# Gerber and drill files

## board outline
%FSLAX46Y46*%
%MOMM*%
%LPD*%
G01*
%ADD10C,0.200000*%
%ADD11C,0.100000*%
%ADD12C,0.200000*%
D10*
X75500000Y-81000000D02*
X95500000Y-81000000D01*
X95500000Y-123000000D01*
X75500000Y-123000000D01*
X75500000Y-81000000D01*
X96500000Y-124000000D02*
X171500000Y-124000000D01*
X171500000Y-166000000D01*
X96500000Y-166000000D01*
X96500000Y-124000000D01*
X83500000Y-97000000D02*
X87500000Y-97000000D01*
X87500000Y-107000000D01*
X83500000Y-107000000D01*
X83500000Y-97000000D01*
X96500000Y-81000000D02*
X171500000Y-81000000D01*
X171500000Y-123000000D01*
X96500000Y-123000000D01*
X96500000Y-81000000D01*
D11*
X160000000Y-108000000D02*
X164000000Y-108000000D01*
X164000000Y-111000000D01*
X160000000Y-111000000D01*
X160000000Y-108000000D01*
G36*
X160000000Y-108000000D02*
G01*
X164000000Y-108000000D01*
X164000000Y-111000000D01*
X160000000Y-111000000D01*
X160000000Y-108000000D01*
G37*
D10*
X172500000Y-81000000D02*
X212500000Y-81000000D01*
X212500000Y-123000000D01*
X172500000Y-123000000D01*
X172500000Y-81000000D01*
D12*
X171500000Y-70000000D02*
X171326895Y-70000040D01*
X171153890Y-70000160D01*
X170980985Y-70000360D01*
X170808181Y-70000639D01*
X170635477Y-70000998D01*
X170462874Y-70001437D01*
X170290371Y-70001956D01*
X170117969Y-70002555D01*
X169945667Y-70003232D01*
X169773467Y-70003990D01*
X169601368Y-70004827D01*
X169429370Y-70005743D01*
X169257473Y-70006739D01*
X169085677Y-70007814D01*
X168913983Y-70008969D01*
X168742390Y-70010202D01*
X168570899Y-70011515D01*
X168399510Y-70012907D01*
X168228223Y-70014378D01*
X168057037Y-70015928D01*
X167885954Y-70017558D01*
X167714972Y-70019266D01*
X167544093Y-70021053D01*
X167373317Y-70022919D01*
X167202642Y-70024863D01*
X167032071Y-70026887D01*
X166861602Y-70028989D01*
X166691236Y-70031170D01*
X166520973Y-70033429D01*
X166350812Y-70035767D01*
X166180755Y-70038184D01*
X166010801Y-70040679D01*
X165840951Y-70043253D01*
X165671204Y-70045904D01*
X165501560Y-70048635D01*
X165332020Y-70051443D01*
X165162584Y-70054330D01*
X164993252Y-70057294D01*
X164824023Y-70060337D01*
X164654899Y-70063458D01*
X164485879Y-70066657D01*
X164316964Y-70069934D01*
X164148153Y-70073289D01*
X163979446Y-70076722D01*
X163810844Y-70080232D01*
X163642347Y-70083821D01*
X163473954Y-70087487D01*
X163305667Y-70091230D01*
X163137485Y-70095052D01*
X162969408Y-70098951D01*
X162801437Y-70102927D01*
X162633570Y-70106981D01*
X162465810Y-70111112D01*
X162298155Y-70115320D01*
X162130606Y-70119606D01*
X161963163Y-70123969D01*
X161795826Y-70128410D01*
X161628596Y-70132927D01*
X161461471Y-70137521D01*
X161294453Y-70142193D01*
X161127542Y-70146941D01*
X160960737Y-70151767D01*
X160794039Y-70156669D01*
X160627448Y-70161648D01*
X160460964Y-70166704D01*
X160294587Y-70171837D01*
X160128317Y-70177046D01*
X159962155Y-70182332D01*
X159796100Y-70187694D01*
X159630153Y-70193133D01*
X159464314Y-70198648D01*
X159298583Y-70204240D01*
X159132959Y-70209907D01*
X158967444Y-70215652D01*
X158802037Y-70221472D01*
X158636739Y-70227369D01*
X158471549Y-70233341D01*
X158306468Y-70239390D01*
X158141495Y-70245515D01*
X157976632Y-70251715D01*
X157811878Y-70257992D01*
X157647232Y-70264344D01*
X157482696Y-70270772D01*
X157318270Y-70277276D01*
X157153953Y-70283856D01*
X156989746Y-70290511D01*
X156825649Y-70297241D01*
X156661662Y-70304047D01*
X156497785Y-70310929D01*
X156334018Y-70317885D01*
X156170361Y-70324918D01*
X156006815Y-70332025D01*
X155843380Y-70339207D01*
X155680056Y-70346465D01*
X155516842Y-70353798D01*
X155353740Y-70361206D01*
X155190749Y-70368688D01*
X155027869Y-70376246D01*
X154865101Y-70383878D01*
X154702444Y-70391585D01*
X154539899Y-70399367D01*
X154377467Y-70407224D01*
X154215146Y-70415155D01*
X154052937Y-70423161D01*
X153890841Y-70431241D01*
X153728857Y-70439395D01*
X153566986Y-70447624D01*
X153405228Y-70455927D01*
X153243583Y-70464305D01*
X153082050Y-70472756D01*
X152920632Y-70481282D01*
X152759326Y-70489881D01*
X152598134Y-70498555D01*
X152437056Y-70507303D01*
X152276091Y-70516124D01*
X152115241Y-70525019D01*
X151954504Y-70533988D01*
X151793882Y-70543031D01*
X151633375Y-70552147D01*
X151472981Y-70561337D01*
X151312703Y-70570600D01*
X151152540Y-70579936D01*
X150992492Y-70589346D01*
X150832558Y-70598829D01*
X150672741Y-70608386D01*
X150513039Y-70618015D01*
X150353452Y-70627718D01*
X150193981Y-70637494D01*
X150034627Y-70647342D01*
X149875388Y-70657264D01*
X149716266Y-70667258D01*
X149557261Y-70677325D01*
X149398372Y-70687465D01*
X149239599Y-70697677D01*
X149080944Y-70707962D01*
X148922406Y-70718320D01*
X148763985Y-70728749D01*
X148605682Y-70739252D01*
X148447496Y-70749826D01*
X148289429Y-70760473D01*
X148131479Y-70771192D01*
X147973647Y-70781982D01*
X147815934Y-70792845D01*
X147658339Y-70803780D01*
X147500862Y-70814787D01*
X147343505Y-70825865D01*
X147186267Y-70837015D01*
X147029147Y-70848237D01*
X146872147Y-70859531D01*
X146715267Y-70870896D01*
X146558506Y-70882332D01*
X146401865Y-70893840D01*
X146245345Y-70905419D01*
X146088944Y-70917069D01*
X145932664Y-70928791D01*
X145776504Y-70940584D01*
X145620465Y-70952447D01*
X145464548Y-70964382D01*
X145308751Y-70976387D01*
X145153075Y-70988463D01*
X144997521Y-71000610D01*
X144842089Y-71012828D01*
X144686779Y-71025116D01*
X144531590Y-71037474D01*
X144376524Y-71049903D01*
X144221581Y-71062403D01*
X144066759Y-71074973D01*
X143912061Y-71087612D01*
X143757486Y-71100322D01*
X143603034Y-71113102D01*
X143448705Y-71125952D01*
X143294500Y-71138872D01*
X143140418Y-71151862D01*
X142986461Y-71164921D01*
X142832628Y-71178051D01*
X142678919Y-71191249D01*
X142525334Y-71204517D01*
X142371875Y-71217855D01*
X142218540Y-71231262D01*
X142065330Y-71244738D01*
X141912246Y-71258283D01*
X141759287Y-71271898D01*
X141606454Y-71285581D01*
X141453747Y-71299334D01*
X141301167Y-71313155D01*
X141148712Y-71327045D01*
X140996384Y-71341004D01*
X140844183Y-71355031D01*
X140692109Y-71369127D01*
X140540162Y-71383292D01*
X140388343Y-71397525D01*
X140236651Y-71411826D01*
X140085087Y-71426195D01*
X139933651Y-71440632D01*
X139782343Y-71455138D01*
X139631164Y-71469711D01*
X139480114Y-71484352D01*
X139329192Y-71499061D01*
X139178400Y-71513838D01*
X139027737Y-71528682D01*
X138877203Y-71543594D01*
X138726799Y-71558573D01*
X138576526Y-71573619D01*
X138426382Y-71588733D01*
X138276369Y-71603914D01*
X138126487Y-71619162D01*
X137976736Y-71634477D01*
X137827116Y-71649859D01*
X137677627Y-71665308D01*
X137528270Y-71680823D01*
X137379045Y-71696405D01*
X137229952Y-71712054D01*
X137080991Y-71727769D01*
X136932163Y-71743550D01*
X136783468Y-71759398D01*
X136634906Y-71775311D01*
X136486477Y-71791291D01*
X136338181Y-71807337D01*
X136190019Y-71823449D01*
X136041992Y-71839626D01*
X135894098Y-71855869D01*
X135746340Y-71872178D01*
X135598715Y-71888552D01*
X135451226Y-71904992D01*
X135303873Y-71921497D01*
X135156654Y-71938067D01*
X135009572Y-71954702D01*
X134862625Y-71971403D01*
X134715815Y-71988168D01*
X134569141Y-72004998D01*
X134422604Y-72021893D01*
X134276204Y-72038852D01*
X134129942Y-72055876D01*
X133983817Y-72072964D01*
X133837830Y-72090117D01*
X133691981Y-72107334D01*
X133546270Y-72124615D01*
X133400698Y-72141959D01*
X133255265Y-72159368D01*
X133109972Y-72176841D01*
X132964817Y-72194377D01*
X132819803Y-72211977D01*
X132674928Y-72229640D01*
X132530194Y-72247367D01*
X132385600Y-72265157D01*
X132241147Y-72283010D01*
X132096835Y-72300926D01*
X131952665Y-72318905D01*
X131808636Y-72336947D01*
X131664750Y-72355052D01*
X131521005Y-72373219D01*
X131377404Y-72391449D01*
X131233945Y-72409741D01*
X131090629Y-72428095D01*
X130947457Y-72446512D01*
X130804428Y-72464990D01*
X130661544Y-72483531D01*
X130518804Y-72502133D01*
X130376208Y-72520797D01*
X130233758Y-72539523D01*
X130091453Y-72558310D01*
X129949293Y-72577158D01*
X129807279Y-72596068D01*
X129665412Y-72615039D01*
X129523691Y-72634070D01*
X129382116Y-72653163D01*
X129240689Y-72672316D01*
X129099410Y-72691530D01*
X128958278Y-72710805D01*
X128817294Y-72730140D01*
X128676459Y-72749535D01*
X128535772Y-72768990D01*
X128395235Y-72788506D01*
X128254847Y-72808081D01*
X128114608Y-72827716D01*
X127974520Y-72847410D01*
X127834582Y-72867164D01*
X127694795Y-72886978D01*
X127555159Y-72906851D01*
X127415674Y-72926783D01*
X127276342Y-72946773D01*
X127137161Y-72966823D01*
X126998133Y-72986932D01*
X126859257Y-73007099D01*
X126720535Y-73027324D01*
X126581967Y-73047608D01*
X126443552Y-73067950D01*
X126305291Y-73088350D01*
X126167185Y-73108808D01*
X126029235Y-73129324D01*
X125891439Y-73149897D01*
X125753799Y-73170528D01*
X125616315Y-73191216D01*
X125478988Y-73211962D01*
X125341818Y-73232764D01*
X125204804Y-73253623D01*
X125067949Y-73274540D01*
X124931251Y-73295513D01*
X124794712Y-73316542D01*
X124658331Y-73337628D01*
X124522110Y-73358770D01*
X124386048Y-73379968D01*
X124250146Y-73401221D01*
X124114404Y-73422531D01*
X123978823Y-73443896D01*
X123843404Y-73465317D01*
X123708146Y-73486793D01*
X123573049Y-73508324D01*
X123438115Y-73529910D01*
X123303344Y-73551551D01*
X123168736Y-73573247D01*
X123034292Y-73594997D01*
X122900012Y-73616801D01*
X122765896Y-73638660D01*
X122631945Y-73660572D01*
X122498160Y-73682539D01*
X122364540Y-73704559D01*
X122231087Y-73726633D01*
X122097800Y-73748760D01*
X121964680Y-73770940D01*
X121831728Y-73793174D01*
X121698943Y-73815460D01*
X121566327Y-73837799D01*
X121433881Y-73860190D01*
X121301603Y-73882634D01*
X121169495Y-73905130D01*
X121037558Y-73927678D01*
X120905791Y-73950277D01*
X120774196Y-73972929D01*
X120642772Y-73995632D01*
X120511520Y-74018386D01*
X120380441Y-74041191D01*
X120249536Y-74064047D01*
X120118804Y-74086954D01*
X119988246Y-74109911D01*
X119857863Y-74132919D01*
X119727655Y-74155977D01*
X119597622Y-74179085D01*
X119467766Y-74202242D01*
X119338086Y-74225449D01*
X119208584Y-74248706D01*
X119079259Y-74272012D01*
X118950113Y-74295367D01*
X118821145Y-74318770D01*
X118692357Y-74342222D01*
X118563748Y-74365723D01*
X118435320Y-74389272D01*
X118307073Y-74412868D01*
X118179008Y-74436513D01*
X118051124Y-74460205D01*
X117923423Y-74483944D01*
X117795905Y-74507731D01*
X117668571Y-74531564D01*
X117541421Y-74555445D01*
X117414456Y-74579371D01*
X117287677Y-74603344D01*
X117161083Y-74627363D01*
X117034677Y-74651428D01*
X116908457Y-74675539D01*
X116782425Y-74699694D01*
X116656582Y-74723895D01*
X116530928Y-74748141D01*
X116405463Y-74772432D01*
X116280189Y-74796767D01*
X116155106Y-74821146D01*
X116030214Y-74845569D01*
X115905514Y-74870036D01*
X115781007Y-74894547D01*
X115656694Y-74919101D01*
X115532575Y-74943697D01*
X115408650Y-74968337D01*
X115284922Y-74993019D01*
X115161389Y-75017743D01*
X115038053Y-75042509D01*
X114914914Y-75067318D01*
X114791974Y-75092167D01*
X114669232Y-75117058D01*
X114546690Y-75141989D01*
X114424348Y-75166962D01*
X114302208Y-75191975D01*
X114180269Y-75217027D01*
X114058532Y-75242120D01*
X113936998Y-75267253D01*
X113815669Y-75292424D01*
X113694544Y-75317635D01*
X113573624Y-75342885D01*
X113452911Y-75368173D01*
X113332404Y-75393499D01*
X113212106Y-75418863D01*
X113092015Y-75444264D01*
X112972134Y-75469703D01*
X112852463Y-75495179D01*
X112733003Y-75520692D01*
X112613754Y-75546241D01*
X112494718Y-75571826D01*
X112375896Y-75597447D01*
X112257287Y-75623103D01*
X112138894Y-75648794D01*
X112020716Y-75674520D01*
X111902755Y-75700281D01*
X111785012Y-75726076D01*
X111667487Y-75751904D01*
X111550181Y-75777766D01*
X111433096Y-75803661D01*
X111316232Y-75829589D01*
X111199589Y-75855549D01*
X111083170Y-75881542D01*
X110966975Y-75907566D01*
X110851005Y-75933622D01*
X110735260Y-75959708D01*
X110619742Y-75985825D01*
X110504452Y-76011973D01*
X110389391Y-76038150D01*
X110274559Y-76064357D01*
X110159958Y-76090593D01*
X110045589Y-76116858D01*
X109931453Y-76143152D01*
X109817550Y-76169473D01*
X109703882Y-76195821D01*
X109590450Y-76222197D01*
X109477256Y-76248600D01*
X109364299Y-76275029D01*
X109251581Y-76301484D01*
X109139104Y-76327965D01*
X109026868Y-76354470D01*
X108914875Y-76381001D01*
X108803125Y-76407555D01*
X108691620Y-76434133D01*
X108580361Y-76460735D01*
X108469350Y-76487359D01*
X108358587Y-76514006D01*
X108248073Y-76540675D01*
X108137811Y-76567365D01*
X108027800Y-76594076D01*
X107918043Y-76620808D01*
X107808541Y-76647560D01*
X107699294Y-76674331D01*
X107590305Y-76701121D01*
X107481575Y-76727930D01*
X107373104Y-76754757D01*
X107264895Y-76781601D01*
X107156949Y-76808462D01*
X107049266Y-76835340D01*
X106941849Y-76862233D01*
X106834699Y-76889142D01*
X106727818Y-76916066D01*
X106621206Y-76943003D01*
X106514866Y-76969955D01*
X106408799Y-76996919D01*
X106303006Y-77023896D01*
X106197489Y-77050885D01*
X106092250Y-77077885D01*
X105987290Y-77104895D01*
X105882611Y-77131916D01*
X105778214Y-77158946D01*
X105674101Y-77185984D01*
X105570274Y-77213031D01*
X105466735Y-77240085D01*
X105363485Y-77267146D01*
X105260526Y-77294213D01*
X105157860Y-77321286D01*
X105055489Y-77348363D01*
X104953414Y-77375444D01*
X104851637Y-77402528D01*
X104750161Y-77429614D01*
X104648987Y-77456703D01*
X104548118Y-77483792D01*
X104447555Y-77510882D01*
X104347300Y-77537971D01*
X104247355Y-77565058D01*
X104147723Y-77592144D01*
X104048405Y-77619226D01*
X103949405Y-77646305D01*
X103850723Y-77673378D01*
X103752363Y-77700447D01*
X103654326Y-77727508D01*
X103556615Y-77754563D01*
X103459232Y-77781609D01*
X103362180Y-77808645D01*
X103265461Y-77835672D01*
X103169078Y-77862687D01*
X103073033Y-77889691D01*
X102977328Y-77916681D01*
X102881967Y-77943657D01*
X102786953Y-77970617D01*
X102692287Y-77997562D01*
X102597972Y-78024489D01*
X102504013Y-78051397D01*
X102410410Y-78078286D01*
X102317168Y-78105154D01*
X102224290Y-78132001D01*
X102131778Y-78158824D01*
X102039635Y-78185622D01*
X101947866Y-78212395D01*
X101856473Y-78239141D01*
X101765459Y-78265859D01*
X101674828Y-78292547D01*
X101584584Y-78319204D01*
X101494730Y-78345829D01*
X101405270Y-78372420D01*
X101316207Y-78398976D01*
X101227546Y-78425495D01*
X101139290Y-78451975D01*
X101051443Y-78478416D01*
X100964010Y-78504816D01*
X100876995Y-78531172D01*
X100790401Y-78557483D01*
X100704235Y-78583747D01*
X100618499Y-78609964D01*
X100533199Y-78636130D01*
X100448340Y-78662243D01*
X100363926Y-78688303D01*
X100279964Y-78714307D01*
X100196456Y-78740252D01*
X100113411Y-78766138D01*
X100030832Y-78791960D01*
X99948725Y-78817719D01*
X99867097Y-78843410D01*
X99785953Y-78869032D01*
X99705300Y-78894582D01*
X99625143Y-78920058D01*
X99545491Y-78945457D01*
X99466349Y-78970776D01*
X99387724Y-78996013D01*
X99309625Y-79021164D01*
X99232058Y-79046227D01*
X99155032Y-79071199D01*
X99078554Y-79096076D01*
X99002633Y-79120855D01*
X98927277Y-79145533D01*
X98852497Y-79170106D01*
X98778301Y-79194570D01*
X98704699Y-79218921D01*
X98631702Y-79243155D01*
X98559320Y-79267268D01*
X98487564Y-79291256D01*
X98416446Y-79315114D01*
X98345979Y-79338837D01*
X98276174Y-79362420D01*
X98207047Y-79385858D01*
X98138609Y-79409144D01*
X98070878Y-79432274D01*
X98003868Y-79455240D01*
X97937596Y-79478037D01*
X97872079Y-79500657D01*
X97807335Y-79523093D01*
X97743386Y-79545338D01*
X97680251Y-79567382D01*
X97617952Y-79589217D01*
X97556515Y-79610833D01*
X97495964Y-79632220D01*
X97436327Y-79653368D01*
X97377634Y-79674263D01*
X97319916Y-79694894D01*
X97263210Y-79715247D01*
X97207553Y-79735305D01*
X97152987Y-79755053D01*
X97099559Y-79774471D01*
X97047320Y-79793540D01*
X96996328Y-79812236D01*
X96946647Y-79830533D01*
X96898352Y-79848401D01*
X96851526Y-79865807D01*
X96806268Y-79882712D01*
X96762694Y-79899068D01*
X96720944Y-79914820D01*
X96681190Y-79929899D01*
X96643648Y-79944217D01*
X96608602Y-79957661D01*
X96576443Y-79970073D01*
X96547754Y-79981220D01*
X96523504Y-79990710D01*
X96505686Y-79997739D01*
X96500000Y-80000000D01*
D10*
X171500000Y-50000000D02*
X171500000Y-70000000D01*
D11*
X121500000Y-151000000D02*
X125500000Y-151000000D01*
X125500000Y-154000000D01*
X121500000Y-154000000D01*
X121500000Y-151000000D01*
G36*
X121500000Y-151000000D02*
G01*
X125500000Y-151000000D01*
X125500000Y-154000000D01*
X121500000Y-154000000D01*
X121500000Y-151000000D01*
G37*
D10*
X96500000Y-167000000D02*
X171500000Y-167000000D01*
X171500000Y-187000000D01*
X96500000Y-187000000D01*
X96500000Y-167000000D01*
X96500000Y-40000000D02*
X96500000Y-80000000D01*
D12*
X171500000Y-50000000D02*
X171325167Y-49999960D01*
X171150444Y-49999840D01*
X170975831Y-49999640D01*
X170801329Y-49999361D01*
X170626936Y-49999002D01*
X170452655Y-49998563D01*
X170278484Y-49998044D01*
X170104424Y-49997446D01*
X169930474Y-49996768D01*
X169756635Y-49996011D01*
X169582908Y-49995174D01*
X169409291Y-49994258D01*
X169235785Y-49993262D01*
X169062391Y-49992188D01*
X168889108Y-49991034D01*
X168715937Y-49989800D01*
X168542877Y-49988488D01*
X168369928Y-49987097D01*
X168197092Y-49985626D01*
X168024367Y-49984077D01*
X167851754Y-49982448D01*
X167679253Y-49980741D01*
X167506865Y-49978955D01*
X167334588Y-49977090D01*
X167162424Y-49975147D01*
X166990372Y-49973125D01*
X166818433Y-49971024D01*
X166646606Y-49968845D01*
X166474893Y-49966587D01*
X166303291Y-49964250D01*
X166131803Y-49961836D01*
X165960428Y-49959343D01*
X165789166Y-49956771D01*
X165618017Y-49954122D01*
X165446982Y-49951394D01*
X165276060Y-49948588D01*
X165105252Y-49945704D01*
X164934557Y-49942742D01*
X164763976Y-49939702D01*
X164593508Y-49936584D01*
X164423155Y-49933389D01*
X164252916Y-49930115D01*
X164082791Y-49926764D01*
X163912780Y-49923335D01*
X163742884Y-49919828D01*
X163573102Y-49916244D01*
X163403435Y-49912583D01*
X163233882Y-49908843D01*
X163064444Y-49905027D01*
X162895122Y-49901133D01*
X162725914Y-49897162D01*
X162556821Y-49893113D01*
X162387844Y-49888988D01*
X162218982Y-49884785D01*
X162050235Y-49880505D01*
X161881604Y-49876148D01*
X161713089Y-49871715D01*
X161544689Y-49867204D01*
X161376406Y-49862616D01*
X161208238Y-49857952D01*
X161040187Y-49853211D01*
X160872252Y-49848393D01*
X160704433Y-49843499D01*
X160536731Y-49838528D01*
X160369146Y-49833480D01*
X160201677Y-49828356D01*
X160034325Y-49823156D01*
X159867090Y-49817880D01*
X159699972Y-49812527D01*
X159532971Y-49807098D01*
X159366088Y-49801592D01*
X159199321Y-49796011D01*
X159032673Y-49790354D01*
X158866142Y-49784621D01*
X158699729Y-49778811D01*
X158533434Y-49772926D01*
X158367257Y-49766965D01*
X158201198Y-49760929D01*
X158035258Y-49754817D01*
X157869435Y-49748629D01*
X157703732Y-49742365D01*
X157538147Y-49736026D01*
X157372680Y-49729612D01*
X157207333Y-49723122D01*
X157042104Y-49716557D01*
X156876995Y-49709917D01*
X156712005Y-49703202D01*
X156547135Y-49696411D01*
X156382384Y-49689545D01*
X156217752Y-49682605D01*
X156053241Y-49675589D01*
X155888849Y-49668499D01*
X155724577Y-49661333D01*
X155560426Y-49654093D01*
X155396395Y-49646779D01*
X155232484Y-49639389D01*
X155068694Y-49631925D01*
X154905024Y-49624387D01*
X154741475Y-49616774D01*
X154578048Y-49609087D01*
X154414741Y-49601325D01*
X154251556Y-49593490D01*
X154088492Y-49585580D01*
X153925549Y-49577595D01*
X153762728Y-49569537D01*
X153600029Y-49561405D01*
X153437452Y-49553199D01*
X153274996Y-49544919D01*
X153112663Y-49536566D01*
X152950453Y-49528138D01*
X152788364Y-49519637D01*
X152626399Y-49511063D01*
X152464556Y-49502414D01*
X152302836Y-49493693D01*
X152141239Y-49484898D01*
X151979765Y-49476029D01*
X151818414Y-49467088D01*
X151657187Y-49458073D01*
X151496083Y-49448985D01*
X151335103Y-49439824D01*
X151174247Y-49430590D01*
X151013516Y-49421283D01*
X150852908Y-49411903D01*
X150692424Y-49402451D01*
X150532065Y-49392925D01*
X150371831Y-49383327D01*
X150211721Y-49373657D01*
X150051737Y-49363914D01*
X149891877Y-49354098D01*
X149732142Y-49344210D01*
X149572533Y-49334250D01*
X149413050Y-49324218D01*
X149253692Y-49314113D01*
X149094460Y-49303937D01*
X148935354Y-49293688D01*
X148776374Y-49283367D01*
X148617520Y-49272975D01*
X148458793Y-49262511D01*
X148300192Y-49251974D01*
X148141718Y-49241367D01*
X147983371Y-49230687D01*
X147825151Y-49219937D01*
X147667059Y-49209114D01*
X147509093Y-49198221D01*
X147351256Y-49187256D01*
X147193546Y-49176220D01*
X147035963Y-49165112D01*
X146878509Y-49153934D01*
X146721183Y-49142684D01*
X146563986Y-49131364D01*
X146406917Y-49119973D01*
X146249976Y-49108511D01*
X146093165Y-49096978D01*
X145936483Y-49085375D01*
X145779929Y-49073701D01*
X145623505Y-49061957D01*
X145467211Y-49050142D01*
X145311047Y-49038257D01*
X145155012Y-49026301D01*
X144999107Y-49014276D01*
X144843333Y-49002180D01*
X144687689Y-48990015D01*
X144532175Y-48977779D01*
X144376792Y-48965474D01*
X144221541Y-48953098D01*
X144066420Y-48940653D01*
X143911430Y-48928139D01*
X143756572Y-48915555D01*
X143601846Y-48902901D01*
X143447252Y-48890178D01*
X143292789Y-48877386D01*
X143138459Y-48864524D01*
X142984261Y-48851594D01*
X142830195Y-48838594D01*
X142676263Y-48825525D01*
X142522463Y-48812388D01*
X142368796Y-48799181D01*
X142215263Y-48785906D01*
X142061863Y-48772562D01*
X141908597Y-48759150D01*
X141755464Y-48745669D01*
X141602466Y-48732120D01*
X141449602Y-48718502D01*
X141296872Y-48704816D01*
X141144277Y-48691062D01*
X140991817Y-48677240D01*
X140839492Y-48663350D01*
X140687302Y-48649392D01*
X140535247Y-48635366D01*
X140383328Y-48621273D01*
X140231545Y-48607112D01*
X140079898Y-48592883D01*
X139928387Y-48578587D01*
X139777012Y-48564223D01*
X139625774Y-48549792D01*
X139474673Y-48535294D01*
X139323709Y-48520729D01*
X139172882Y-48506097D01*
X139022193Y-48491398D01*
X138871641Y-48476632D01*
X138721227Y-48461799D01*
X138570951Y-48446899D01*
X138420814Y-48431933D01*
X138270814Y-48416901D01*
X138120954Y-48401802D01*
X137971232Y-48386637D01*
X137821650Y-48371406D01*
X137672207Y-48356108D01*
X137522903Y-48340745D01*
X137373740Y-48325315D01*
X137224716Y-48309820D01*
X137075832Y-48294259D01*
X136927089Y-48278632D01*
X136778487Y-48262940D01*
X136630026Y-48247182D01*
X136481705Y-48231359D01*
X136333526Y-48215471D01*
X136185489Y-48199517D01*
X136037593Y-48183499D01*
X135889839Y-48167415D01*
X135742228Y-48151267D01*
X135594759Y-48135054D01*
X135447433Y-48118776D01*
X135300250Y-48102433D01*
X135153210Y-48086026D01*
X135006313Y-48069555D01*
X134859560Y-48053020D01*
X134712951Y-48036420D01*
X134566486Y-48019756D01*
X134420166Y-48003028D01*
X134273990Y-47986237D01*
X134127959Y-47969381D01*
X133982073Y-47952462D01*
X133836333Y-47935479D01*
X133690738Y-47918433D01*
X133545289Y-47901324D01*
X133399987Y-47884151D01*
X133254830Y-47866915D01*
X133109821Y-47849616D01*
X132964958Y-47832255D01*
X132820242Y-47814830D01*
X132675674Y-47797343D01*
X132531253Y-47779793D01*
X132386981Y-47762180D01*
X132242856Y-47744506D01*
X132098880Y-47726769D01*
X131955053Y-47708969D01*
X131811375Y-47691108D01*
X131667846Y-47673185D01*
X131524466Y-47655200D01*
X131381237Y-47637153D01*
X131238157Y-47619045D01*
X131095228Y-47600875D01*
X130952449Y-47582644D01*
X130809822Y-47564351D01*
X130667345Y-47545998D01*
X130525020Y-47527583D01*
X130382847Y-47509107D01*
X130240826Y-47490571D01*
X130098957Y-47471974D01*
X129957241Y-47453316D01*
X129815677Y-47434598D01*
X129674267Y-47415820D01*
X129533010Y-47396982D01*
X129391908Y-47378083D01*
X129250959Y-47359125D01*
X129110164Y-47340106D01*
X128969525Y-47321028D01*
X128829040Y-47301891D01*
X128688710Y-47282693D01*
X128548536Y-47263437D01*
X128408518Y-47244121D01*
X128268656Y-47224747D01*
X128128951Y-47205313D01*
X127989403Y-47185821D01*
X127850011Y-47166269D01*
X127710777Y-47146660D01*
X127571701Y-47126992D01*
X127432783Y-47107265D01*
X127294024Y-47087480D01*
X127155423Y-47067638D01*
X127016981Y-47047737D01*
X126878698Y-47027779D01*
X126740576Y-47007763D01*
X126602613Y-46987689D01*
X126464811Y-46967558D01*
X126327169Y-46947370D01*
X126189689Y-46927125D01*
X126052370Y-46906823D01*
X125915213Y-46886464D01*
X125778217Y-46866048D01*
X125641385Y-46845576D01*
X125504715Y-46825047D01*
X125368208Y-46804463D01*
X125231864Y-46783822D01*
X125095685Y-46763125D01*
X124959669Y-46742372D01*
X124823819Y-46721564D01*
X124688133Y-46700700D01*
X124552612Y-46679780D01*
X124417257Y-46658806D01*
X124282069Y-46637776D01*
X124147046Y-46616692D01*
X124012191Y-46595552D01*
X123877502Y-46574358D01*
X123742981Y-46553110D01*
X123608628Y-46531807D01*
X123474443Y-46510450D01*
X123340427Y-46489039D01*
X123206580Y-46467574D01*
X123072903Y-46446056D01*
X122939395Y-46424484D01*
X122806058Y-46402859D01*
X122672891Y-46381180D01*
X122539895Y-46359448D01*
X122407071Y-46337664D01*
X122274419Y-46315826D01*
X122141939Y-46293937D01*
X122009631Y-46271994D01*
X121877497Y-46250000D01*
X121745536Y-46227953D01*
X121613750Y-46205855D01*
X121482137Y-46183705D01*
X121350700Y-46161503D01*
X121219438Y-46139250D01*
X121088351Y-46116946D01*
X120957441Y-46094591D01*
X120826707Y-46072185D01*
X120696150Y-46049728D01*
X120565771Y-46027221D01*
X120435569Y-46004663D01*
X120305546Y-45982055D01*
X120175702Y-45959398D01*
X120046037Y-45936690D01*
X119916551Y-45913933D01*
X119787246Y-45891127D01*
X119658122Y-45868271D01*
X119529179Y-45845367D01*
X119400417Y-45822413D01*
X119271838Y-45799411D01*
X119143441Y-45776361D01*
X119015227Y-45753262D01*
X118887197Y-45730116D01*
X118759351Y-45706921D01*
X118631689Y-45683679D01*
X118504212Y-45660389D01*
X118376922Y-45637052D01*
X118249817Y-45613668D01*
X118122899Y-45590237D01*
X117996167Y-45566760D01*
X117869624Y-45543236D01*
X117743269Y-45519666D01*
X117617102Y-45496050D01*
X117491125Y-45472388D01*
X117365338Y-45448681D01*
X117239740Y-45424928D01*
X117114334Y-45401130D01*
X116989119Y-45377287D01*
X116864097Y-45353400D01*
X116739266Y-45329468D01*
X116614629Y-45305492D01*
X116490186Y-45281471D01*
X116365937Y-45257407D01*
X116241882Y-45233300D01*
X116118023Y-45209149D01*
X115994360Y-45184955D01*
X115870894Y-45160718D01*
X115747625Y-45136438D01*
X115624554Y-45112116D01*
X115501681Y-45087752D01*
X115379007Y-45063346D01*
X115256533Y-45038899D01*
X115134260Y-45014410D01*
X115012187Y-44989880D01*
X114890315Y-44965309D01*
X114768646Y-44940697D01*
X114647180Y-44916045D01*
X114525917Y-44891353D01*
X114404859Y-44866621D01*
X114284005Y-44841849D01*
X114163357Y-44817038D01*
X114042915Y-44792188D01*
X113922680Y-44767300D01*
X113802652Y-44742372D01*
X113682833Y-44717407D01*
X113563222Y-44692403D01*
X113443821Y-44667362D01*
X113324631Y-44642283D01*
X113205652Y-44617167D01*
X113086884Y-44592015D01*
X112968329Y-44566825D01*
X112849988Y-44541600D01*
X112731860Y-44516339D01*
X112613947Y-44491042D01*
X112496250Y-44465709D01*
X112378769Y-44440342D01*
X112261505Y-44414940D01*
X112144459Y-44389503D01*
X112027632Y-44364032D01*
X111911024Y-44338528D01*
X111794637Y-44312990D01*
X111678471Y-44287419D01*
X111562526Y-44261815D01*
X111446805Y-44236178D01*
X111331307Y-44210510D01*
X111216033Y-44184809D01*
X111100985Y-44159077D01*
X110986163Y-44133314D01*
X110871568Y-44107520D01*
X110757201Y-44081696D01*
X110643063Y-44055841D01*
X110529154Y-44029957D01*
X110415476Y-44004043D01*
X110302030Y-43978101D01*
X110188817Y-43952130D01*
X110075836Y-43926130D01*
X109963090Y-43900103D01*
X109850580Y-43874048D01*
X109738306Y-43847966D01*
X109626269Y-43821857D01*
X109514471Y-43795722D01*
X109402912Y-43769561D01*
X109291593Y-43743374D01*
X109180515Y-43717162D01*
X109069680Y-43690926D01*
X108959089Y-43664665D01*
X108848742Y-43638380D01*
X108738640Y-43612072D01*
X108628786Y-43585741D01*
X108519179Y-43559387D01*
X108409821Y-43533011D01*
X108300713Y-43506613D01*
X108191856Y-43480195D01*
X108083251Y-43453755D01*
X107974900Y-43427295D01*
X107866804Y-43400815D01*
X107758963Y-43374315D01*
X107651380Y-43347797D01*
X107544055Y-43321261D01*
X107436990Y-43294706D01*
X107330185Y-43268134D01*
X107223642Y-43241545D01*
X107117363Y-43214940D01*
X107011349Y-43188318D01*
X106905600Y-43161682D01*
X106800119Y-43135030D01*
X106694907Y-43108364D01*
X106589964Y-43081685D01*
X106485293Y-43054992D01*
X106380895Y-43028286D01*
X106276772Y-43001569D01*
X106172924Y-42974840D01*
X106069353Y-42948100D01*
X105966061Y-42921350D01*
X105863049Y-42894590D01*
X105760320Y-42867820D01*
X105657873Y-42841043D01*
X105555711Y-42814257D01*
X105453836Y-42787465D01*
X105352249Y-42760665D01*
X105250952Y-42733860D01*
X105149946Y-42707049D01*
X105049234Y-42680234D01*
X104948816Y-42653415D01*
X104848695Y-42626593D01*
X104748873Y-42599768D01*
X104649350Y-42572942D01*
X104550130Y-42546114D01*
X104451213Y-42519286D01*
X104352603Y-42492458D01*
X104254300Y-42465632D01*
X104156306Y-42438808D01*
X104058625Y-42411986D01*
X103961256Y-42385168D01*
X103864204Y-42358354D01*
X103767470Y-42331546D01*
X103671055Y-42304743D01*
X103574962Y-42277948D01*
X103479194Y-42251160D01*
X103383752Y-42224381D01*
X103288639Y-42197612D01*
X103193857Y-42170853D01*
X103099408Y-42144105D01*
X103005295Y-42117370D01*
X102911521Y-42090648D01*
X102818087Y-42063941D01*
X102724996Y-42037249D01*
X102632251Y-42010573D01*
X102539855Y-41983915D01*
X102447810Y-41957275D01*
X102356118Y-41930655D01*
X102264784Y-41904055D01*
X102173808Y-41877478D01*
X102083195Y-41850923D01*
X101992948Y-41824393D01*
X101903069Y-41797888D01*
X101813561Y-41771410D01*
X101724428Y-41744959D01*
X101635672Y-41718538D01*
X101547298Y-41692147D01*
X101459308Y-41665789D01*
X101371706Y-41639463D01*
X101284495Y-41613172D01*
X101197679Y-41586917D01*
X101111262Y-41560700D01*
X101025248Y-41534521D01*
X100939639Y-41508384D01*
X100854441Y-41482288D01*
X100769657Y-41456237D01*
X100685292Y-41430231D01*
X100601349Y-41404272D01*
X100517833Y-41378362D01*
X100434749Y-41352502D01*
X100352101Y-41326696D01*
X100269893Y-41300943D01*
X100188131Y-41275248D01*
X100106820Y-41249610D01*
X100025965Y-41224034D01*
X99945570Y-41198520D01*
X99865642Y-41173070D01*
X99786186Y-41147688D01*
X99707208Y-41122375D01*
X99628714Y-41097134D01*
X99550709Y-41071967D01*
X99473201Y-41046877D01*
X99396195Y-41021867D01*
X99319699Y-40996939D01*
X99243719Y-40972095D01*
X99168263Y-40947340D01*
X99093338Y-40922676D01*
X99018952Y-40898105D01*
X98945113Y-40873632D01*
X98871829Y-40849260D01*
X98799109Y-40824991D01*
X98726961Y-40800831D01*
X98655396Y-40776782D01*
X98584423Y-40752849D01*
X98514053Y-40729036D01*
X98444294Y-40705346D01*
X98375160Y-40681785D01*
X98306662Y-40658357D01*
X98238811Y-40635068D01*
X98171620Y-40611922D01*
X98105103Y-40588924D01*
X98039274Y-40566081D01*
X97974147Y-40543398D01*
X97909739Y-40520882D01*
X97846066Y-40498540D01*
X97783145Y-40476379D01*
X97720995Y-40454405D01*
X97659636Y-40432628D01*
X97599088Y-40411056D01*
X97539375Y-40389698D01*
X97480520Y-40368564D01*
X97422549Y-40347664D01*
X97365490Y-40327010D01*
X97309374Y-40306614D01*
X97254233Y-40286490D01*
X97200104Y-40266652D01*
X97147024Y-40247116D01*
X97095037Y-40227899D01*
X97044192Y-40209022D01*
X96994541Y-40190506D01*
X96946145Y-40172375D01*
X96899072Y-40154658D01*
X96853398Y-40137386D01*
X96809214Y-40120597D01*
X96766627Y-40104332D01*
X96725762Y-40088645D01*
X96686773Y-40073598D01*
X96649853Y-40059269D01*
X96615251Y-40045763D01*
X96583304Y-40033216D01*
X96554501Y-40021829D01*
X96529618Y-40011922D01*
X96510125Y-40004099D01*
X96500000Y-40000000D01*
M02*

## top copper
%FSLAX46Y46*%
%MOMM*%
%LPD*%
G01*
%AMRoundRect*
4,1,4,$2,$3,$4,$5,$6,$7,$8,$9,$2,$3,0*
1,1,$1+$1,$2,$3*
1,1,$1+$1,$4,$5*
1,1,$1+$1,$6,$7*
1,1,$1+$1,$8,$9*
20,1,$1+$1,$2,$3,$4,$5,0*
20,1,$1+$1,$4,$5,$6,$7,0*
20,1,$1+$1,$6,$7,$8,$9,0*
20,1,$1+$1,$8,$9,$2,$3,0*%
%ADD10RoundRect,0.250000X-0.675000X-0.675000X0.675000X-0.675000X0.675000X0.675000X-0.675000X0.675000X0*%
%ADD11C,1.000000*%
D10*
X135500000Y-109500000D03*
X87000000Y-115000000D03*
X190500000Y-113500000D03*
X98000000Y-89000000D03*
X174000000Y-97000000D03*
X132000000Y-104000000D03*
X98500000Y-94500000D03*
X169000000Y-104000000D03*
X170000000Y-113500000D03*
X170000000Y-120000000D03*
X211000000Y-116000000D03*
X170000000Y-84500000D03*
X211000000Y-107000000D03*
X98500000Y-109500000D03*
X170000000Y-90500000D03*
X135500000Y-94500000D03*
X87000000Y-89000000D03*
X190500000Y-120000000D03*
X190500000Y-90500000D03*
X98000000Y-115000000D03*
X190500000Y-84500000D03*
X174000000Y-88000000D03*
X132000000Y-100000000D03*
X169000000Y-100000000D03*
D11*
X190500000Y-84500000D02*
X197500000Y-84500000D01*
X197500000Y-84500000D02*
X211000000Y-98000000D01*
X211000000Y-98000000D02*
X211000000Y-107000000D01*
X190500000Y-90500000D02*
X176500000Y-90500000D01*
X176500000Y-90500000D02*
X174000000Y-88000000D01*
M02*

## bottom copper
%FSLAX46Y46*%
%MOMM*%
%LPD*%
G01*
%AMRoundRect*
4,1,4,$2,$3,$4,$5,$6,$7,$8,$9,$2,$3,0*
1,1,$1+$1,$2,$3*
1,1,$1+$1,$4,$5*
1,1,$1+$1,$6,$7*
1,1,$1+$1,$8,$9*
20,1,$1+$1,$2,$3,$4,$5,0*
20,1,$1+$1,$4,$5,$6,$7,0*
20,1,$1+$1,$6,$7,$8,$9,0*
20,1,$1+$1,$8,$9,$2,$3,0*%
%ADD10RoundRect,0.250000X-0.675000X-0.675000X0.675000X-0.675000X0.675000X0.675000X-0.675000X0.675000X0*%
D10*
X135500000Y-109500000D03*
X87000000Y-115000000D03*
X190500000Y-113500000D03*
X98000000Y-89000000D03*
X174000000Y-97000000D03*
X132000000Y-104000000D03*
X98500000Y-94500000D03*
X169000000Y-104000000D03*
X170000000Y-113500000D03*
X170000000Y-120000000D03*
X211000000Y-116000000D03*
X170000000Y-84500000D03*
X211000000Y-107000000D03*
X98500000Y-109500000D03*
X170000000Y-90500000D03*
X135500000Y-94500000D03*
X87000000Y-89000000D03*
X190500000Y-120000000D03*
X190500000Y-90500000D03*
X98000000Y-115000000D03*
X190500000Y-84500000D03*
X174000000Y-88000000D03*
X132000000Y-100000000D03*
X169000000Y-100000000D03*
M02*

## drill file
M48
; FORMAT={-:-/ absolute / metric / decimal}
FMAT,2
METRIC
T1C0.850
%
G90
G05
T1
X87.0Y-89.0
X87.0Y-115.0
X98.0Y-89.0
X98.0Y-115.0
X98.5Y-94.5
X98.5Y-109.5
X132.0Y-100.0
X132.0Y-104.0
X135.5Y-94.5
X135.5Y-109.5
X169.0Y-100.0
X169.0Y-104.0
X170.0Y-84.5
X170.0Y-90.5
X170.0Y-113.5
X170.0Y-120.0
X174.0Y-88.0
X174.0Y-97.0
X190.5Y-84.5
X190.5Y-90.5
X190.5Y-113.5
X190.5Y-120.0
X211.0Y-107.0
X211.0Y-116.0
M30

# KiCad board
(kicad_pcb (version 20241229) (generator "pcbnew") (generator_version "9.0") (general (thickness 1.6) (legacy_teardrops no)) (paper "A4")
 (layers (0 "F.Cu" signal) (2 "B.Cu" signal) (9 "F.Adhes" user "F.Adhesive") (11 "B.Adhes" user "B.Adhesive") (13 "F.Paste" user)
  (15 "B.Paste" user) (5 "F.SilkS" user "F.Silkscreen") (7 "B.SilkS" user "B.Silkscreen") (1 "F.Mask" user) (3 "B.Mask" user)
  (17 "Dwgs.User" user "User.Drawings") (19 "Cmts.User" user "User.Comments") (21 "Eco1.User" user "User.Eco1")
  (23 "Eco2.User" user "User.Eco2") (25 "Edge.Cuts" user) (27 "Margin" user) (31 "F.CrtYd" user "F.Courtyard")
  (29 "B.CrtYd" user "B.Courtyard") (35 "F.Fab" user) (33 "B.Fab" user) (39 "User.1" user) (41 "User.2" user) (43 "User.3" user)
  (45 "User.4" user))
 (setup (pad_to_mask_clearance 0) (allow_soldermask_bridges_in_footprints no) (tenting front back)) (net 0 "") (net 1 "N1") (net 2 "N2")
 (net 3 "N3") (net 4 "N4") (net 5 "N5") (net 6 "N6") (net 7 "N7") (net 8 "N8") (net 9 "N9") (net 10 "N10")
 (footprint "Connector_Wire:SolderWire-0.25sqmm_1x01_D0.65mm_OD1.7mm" (layer "F.Cu") (at 135.5 109.5)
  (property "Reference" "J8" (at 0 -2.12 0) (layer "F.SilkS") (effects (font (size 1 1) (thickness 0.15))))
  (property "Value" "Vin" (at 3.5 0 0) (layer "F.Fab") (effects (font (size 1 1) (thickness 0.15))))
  (pad "1" thru_hole roundrect (at 0 0) (size 1.85 1.85) (drill 0.85) (layers "*.Cu" "*.Mask") (remove_unused_layers no)
   (roundrect_rratio 0.135135) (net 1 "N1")))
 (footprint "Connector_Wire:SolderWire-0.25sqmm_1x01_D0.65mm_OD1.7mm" (layer "F.Cu") (at 87 115)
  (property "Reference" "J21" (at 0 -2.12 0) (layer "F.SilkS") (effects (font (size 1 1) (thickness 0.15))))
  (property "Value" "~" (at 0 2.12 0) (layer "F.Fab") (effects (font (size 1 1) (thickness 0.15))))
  (pad "1" thru_hole roundrect (at 0 0) (size 1.85 1.85) (drill 0.85) (layers "*.Cu" "*.Mask") (remove_unused_layers no)
   (roundrect_rratio 0.135135) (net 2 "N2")))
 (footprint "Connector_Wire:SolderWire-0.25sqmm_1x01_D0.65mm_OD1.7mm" (layer "F.Cu") (at 190.5 113.5)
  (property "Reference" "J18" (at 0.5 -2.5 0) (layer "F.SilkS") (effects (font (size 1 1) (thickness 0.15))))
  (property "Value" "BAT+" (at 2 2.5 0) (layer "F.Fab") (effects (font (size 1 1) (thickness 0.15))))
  (pad "1" thru_hole roundrect (at 0 0) (size 1.85 1.85) (drill 0.85) (layers "*.Cu" "*.Mask") (remove_unused_layers no)
   (roundrect_rratio 0.135135) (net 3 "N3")))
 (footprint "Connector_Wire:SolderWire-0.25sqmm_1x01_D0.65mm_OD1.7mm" (layer "F.Cu") (at 98 89)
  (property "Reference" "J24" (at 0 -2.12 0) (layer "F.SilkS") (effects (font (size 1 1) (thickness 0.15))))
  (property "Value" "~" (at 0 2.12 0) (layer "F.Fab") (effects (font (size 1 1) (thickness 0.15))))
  (pad "1" thru_hole roundrect (at 0 0) (size 1.85 1.85) (drill 0.85) (layers "*.Cu" "*.Mask") (remove_unused_layers no)
   (roundrect_rratio 0.135135) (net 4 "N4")))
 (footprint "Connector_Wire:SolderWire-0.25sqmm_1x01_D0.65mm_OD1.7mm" (layer "F.Cu") (at 174 97)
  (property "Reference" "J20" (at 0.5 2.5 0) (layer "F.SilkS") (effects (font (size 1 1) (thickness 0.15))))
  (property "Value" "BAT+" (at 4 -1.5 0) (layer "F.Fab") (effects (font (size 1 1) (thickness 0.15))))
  (pad "1" thru_hole roundrect (at 0 0) (size 1.85 1.85) (drill 0.85) (layers "*.Cu" "*.Mask") (remove_unused_layers no)
   (roundrect_rratio 0.135135) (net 3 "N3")))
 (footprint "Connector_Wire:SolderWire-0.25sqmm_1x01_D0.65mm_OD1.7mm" (layer "F.Cu") (at 132 104)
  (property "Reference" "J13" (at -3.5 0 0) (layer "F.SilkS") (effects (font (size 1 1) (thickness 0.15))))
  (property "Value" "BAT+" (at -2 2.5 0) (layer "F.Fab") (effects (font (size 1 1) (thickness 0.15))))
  (pad "1" thru_hole roundrect (at 0 0) (size 1.85 1.85) (drill 0.85) (layers "*.Cu" "*.Mask") (remove_unused_layers no)
   (roundrect_rratio 0.135135) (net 3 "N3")))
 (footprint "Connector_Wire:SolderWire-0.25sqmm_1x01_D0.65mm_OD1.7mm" (layer "F.Cu") (at 98.5 94.5)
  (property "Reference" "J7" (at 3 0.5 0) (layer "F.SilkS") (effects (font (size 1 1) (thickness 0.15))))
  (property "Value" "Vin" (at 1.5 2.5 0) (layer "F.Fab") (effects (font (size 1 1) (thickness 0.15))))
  (pad "1" thru_hole roundrect (at 0 0) (size 1.85 1.85) (drill 0.85) (layers "*.Cu" "*.Mask") (remove_unused_layers no)
   (roundrect_rratio 0.135135) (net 1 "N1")))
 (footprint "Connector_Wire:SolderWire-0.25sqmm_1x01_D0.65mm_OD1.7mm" (layer "F.Cu") (at 169 104)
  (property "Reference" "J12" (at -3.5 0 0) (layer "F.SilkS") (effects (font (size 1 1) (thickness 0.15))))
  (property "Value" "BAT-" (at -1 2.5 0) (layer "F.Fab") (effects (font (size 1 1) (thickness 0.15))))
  (pad "1" thru_hole roundrect (at 0 0) (size 1.85 1.85) (drill 0.85) (layers "*.Cu" "*.Mask") (remove_unused_layers no)
   (roundrect_rratio 0.135135) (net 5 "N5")))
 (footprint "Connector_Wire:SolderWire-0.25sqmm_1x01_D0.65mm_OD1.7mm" (layer "F.Cu") (at 170 113.5)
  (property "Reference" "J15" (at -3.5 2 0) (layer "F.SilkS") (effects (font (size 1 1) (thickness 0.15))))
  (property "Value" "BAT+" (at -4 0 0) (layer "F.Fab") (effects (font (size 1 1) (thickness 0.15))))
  (pad "1" thru_hole roundrect (at 0 0) (size 1.85 1.85) (drill 0.85) (layers "*.Cu" "*.Mask") (remove_unused_layers no)
   (roundrect_rratio 0.135135) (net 3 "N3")))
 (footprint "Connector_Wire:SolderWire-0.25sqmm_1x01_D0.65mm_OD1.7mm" (layer "F.Cu") (at 170 120)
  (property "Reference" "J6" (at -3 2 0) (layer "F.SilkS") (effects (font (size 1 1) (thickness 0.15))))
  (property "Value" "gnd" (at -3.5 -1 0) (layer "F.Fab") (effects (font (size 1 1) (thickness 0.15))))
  (pad "1" thru_hole roundrect (at 0 0) (size 1.85 1.85) (drill 0.85) (layers "*.Cu" "*.Mask") (remove_unused_layers no)
   (roundrect_rratio 0.135135) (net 5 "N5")))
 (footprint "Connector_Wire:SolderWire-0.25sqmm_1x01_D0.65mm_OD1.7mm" (layer "F.Cu") (at 211 116)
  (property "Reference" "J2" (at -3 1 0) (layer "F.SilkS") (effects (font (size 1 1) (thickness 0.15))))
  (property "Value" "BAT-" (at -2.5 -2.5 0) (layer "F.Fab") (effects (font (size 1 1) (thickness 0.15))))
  (pad "1" thru_hole roundrect (at 0 0) (size 1.85 1.85) (drill 0.85) (layers "*.Cu" "*.Mask") (remove_unused_layers no)
   (roundrect_rratio 0.135135) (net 5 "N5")))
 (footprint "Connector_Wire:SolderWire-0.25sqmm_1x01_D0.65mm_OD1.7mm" (layer "F.Cu") (at 170 84.5)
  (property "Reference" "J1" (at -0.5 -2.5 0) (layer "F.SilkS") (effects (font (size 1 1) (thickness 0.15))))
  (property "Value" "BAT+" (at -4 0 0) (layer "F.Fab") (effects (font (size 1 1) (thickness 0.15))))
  (pad "1" thru_hole roundrect (at 0 0) (size 1.85 1.85) (drill 0.85) (layers "*.Cu" "*.Mask") (remove_unused_layers no)
   (roundrect_rratio 0.135135) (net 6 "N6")))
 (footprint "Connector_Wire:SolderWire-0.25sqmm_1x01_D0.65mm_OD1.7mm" (layer "F.Cu") (at 211 107)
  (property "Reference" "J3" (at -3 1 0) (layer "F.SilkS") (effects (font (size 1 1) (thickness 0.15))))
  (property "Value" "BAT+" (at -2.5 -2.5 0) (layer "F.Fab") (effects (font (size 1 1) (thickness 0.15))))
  (pad "1" thru_hole roundrect (at 0 0) (size 1.85 1.85) (drill 0.85) (layers "*.Cu" "*.Mask") (remove_unused_layers no)
   (roundrect_rratio 0.135135) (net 6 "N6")))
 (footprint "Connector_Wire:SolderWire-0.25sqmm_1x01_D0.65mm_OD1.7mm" (layer "F.Cu") (at 98.5 109.5)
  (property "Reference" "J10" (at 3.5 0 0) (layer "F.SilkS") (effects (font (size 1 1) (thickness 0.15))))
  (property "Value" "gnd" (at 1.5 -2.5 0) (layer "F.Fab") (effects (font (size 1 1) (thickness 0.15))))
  (pad "1" thru_hole roundrect (at 0 0) (size 1.85 1.85) (drill 0.85) (layers "*.Cu" "*.Mask") (remove_unused_layers no)
   (roundrect_rratio 0.135135) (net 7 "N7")))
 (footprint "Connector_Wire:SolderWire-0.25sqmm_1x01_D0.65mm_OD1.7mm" (layer "F.Cu") (at 170 90.5)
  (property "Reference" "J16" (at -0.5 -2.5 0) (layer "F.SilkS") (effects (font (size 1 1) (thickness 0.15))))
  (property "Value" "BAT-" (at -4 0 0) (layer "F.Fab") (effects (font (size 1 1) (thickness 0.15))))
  (pad "1" thru_hole roundrect (at 0 0) (size 1.85 1.85) (drill 0.85) (layers "*.Cu" "*.Mask") (remove_unused_layers no)
   (roundrect_rratio 0.135135) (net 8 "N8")))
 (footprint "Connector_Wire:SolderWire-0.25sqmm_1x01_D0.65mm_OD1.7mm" (layer "F.Cu") (at 135.5 94.5)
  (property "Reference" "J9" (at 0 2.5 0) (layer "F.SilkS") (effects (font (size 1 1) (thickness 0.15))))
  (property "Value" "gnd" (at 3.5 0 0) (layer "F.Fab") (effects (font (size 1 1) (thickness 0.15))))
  (pad "1" thru_hole roundrect (at 0 0) (size 1.85 1.85) (drill 0.85) (layers "*.Cu" "*.Mask") (remove_unused_layers no)
   (roundrect_rratio 0.135135) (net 7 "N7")))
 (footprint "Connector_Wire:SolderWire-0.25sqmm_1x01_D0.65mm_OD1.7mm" (layer "F.Cu") (at 87 89)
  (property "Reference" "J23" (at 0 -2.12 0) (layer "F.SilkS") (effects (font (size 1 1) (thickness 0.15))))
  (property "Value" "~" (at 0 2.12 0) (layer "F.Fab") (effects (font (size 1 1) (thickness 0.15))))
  (pad "1" thru_hole roundrect (at 0 0) (size 1.85 1.85) (drill 0.85) (layers "*.Cu" "*.Mask") (remove_unused_layers no)
   (roundrect_rratio 0.135135) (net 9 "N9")))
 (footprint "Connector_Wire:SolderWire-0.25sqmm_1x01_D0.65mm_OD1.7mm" (layer "F.Cu") (at 190.5 120)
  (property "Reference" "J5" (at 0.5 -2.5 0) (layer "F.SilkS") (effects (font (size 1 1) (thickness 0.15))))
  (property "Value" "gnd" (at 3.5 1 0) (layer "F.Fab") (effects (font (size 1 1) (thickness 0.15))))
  (pad "1" thru_hole roundrect (at 0 0) (size 1.85 1.85) (drill 0.85) (layers "*.Cu" "*.Mask") (remove_unused_layers no)
   (roundrect_rratio 0.135135) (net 5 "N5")))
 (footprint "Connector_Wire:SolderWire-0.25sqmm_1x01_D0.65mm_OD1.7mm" (layer "F.Cu") (at 190.5 90.5)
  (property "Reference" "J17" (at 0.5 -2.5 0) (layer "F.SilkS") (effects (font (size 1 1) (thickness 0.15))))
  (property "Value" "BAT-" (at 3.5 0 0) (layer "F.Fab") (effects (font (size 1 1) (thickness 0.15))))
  (pad "1" thru_hole roundrect (at 0 0) (size 1.85 1.85) (drill 0.85) (layers "*.Cu" "*.Mask") (remove_unused_layers no)
   (roundrect_rratio 0.135135) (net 8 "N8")))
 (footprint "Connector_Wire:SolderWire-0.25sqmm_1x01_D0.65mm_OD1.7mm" (layer "F.Cu") (at 98 115)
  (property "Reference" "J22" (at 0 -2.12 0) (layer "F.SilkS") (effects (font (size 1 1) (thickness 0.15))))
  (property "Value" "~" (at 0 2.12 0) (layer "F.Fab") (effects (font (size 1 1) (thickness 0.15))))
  (pad "1" thru_hole roundrect (at 0 0) (size 1.85 1.85) (drill 0.85) (layers "*.Cu" "*.Mask") (remove_unused_layers no)
   (roundrect_rratio 0.135135) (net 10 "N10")))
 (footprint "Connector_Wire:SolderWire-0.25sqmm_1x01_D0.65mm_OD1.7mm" (layer "F.Cu") (at 190.5 84.5)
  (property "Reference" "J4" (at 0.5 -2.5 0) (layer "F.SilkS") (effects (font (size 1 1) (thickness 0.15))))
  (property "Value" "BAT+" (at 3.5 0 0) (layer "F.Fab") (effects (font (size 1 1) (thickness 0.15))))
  (pad "1" thru_hole roundrect (at 0 0) (size 1.85 1.85) (drill 0.85) (layers "*.Cu" "*.Mask") (remove_unused_layers no)
   (roundrect_rratio 0.135135) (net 6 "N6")))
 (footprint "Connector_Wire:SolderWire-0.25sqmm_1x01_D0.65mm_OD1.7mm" (layer "F.Cu") (at 174 88)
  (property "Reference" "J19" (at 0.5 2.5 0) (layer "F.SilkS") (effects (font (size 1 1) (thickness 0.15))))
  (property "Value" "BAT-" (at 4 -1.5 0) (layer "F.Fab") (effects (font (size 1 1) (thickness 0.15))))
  (pad "1" thru_hole roundrect (at 0 0) (size 1.85 1.85) (drill 0.85) (layers "*.Cu" "*.Mask") (remove_unused_layers no)
   (roundrect_rratio 0.135135) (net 8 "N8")))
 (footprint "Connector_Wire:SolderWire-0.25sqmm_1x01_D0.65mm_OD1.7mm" (layer "F.Cu") (at 132 100)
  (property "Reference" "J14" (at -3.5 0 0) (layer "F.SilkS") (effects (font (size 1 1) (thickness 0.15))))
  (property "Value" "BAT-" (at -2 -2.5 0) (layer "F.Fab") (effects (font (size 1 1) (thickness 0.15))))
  (pad "1" thru_hole roundrect (at 0 0) (size 1.85 1.85) (drill 0.85) (layers "*.Cu" "*.Mask") (remove_unused_layers no)
   (roundrect_rratio 0.135135) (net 8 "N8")))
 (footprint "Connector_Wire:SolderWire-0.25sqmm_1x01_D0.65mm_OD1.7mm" (layer "F.Cu") (at 169 100)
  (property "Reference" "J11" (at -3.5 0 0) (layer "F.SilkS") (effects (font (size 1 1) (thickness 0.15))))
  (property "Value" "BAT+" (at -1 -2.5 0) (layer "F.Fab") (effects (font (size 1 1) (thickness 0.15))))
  (pad "1" thru_hole roundrect (at 0 0) (size 1.85 1.85) (drill 0.85) (layers "*.Cu" "*.Mask") (remove_unused_layers no)
   (roundrect_rratio 0.135135) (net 6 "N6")))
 (gr_rect (start 75.5 81) (end 95.5 123) (stroke (width 0.2) (type solid)) (fill no) (layer "Edge.Cuts"))
 (gr_rect (start 96.5 124) (end 171.5 166) (stroke (width 0.2) (type solid)) (fill no) (layer "Edge.Cuts"))
 (gr_rect (start 83.5 97) (end 87.5 107) (stroke (width 0.2) (type solid)) (fill no) (layer "Edge.Cuts"))
 (gr_rect (start 96.5 81) (end 171.5 123) (stroke (width 0.2) (type solid)) (fill no) (layer "Edge.Cuts"))
 (gr_rect (start 160 108) (end 164 111) (stroke (width 0.1) (type solid)) (fill yes) (layer "Edge.Cuts"))
 (gr_rect (start 172.5 81) (end 212.5 123) (stroke (width 0.2) (type solid)) (fill no) (layer "Edge.Cuts"))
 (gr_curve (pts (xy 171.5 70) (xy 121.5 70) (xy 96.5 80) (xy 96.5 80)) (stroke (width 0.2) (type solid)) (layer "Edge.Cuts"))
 (gr_line (start 171.5 50) (end 171.5 70) (stroke (width 0.2) (type solid)) (layer "Edge.Cuts"))
 (gr_rect (start 121.5 151) (end 125.5 154) (stroke (width 0.1) (type solid)) (fill yes) (layer "Edge.Cuts"))
 (gr_rect (start 96.5 167) (end 171.5 187) (stroke (width 0.2) (type solid)) (fill no) (layer "Edge.Cuts"))
 (gr_line (start 96.5 40) (end 96.5 80) (stroke (width 0.2) (type solid)) (layer "Edge.Cuts"))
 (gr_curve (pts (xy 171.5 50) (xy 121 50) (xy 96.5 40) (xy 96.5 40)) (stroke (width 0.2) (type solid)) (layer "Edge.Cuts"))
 (segment (start 190.5 84.5) (end 197.5 84.5) (width 1) (layer "F.Cu") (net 6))
 (segment (start 197.5 84.5) (end 211 98) (width 1) (layer "F.Cu") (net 6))
 (segment (start 211 98) (end 211 107) (width 1) (layer "F.Cu") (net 6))
 (segment (start 190.5 90.5) (end 176.5 90.5) (width 1) (layer "F.Cu") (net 8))
 (segment (start 176.5 90.5) (end 174 88) (width 1) (layer "F.Cu") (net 8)))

